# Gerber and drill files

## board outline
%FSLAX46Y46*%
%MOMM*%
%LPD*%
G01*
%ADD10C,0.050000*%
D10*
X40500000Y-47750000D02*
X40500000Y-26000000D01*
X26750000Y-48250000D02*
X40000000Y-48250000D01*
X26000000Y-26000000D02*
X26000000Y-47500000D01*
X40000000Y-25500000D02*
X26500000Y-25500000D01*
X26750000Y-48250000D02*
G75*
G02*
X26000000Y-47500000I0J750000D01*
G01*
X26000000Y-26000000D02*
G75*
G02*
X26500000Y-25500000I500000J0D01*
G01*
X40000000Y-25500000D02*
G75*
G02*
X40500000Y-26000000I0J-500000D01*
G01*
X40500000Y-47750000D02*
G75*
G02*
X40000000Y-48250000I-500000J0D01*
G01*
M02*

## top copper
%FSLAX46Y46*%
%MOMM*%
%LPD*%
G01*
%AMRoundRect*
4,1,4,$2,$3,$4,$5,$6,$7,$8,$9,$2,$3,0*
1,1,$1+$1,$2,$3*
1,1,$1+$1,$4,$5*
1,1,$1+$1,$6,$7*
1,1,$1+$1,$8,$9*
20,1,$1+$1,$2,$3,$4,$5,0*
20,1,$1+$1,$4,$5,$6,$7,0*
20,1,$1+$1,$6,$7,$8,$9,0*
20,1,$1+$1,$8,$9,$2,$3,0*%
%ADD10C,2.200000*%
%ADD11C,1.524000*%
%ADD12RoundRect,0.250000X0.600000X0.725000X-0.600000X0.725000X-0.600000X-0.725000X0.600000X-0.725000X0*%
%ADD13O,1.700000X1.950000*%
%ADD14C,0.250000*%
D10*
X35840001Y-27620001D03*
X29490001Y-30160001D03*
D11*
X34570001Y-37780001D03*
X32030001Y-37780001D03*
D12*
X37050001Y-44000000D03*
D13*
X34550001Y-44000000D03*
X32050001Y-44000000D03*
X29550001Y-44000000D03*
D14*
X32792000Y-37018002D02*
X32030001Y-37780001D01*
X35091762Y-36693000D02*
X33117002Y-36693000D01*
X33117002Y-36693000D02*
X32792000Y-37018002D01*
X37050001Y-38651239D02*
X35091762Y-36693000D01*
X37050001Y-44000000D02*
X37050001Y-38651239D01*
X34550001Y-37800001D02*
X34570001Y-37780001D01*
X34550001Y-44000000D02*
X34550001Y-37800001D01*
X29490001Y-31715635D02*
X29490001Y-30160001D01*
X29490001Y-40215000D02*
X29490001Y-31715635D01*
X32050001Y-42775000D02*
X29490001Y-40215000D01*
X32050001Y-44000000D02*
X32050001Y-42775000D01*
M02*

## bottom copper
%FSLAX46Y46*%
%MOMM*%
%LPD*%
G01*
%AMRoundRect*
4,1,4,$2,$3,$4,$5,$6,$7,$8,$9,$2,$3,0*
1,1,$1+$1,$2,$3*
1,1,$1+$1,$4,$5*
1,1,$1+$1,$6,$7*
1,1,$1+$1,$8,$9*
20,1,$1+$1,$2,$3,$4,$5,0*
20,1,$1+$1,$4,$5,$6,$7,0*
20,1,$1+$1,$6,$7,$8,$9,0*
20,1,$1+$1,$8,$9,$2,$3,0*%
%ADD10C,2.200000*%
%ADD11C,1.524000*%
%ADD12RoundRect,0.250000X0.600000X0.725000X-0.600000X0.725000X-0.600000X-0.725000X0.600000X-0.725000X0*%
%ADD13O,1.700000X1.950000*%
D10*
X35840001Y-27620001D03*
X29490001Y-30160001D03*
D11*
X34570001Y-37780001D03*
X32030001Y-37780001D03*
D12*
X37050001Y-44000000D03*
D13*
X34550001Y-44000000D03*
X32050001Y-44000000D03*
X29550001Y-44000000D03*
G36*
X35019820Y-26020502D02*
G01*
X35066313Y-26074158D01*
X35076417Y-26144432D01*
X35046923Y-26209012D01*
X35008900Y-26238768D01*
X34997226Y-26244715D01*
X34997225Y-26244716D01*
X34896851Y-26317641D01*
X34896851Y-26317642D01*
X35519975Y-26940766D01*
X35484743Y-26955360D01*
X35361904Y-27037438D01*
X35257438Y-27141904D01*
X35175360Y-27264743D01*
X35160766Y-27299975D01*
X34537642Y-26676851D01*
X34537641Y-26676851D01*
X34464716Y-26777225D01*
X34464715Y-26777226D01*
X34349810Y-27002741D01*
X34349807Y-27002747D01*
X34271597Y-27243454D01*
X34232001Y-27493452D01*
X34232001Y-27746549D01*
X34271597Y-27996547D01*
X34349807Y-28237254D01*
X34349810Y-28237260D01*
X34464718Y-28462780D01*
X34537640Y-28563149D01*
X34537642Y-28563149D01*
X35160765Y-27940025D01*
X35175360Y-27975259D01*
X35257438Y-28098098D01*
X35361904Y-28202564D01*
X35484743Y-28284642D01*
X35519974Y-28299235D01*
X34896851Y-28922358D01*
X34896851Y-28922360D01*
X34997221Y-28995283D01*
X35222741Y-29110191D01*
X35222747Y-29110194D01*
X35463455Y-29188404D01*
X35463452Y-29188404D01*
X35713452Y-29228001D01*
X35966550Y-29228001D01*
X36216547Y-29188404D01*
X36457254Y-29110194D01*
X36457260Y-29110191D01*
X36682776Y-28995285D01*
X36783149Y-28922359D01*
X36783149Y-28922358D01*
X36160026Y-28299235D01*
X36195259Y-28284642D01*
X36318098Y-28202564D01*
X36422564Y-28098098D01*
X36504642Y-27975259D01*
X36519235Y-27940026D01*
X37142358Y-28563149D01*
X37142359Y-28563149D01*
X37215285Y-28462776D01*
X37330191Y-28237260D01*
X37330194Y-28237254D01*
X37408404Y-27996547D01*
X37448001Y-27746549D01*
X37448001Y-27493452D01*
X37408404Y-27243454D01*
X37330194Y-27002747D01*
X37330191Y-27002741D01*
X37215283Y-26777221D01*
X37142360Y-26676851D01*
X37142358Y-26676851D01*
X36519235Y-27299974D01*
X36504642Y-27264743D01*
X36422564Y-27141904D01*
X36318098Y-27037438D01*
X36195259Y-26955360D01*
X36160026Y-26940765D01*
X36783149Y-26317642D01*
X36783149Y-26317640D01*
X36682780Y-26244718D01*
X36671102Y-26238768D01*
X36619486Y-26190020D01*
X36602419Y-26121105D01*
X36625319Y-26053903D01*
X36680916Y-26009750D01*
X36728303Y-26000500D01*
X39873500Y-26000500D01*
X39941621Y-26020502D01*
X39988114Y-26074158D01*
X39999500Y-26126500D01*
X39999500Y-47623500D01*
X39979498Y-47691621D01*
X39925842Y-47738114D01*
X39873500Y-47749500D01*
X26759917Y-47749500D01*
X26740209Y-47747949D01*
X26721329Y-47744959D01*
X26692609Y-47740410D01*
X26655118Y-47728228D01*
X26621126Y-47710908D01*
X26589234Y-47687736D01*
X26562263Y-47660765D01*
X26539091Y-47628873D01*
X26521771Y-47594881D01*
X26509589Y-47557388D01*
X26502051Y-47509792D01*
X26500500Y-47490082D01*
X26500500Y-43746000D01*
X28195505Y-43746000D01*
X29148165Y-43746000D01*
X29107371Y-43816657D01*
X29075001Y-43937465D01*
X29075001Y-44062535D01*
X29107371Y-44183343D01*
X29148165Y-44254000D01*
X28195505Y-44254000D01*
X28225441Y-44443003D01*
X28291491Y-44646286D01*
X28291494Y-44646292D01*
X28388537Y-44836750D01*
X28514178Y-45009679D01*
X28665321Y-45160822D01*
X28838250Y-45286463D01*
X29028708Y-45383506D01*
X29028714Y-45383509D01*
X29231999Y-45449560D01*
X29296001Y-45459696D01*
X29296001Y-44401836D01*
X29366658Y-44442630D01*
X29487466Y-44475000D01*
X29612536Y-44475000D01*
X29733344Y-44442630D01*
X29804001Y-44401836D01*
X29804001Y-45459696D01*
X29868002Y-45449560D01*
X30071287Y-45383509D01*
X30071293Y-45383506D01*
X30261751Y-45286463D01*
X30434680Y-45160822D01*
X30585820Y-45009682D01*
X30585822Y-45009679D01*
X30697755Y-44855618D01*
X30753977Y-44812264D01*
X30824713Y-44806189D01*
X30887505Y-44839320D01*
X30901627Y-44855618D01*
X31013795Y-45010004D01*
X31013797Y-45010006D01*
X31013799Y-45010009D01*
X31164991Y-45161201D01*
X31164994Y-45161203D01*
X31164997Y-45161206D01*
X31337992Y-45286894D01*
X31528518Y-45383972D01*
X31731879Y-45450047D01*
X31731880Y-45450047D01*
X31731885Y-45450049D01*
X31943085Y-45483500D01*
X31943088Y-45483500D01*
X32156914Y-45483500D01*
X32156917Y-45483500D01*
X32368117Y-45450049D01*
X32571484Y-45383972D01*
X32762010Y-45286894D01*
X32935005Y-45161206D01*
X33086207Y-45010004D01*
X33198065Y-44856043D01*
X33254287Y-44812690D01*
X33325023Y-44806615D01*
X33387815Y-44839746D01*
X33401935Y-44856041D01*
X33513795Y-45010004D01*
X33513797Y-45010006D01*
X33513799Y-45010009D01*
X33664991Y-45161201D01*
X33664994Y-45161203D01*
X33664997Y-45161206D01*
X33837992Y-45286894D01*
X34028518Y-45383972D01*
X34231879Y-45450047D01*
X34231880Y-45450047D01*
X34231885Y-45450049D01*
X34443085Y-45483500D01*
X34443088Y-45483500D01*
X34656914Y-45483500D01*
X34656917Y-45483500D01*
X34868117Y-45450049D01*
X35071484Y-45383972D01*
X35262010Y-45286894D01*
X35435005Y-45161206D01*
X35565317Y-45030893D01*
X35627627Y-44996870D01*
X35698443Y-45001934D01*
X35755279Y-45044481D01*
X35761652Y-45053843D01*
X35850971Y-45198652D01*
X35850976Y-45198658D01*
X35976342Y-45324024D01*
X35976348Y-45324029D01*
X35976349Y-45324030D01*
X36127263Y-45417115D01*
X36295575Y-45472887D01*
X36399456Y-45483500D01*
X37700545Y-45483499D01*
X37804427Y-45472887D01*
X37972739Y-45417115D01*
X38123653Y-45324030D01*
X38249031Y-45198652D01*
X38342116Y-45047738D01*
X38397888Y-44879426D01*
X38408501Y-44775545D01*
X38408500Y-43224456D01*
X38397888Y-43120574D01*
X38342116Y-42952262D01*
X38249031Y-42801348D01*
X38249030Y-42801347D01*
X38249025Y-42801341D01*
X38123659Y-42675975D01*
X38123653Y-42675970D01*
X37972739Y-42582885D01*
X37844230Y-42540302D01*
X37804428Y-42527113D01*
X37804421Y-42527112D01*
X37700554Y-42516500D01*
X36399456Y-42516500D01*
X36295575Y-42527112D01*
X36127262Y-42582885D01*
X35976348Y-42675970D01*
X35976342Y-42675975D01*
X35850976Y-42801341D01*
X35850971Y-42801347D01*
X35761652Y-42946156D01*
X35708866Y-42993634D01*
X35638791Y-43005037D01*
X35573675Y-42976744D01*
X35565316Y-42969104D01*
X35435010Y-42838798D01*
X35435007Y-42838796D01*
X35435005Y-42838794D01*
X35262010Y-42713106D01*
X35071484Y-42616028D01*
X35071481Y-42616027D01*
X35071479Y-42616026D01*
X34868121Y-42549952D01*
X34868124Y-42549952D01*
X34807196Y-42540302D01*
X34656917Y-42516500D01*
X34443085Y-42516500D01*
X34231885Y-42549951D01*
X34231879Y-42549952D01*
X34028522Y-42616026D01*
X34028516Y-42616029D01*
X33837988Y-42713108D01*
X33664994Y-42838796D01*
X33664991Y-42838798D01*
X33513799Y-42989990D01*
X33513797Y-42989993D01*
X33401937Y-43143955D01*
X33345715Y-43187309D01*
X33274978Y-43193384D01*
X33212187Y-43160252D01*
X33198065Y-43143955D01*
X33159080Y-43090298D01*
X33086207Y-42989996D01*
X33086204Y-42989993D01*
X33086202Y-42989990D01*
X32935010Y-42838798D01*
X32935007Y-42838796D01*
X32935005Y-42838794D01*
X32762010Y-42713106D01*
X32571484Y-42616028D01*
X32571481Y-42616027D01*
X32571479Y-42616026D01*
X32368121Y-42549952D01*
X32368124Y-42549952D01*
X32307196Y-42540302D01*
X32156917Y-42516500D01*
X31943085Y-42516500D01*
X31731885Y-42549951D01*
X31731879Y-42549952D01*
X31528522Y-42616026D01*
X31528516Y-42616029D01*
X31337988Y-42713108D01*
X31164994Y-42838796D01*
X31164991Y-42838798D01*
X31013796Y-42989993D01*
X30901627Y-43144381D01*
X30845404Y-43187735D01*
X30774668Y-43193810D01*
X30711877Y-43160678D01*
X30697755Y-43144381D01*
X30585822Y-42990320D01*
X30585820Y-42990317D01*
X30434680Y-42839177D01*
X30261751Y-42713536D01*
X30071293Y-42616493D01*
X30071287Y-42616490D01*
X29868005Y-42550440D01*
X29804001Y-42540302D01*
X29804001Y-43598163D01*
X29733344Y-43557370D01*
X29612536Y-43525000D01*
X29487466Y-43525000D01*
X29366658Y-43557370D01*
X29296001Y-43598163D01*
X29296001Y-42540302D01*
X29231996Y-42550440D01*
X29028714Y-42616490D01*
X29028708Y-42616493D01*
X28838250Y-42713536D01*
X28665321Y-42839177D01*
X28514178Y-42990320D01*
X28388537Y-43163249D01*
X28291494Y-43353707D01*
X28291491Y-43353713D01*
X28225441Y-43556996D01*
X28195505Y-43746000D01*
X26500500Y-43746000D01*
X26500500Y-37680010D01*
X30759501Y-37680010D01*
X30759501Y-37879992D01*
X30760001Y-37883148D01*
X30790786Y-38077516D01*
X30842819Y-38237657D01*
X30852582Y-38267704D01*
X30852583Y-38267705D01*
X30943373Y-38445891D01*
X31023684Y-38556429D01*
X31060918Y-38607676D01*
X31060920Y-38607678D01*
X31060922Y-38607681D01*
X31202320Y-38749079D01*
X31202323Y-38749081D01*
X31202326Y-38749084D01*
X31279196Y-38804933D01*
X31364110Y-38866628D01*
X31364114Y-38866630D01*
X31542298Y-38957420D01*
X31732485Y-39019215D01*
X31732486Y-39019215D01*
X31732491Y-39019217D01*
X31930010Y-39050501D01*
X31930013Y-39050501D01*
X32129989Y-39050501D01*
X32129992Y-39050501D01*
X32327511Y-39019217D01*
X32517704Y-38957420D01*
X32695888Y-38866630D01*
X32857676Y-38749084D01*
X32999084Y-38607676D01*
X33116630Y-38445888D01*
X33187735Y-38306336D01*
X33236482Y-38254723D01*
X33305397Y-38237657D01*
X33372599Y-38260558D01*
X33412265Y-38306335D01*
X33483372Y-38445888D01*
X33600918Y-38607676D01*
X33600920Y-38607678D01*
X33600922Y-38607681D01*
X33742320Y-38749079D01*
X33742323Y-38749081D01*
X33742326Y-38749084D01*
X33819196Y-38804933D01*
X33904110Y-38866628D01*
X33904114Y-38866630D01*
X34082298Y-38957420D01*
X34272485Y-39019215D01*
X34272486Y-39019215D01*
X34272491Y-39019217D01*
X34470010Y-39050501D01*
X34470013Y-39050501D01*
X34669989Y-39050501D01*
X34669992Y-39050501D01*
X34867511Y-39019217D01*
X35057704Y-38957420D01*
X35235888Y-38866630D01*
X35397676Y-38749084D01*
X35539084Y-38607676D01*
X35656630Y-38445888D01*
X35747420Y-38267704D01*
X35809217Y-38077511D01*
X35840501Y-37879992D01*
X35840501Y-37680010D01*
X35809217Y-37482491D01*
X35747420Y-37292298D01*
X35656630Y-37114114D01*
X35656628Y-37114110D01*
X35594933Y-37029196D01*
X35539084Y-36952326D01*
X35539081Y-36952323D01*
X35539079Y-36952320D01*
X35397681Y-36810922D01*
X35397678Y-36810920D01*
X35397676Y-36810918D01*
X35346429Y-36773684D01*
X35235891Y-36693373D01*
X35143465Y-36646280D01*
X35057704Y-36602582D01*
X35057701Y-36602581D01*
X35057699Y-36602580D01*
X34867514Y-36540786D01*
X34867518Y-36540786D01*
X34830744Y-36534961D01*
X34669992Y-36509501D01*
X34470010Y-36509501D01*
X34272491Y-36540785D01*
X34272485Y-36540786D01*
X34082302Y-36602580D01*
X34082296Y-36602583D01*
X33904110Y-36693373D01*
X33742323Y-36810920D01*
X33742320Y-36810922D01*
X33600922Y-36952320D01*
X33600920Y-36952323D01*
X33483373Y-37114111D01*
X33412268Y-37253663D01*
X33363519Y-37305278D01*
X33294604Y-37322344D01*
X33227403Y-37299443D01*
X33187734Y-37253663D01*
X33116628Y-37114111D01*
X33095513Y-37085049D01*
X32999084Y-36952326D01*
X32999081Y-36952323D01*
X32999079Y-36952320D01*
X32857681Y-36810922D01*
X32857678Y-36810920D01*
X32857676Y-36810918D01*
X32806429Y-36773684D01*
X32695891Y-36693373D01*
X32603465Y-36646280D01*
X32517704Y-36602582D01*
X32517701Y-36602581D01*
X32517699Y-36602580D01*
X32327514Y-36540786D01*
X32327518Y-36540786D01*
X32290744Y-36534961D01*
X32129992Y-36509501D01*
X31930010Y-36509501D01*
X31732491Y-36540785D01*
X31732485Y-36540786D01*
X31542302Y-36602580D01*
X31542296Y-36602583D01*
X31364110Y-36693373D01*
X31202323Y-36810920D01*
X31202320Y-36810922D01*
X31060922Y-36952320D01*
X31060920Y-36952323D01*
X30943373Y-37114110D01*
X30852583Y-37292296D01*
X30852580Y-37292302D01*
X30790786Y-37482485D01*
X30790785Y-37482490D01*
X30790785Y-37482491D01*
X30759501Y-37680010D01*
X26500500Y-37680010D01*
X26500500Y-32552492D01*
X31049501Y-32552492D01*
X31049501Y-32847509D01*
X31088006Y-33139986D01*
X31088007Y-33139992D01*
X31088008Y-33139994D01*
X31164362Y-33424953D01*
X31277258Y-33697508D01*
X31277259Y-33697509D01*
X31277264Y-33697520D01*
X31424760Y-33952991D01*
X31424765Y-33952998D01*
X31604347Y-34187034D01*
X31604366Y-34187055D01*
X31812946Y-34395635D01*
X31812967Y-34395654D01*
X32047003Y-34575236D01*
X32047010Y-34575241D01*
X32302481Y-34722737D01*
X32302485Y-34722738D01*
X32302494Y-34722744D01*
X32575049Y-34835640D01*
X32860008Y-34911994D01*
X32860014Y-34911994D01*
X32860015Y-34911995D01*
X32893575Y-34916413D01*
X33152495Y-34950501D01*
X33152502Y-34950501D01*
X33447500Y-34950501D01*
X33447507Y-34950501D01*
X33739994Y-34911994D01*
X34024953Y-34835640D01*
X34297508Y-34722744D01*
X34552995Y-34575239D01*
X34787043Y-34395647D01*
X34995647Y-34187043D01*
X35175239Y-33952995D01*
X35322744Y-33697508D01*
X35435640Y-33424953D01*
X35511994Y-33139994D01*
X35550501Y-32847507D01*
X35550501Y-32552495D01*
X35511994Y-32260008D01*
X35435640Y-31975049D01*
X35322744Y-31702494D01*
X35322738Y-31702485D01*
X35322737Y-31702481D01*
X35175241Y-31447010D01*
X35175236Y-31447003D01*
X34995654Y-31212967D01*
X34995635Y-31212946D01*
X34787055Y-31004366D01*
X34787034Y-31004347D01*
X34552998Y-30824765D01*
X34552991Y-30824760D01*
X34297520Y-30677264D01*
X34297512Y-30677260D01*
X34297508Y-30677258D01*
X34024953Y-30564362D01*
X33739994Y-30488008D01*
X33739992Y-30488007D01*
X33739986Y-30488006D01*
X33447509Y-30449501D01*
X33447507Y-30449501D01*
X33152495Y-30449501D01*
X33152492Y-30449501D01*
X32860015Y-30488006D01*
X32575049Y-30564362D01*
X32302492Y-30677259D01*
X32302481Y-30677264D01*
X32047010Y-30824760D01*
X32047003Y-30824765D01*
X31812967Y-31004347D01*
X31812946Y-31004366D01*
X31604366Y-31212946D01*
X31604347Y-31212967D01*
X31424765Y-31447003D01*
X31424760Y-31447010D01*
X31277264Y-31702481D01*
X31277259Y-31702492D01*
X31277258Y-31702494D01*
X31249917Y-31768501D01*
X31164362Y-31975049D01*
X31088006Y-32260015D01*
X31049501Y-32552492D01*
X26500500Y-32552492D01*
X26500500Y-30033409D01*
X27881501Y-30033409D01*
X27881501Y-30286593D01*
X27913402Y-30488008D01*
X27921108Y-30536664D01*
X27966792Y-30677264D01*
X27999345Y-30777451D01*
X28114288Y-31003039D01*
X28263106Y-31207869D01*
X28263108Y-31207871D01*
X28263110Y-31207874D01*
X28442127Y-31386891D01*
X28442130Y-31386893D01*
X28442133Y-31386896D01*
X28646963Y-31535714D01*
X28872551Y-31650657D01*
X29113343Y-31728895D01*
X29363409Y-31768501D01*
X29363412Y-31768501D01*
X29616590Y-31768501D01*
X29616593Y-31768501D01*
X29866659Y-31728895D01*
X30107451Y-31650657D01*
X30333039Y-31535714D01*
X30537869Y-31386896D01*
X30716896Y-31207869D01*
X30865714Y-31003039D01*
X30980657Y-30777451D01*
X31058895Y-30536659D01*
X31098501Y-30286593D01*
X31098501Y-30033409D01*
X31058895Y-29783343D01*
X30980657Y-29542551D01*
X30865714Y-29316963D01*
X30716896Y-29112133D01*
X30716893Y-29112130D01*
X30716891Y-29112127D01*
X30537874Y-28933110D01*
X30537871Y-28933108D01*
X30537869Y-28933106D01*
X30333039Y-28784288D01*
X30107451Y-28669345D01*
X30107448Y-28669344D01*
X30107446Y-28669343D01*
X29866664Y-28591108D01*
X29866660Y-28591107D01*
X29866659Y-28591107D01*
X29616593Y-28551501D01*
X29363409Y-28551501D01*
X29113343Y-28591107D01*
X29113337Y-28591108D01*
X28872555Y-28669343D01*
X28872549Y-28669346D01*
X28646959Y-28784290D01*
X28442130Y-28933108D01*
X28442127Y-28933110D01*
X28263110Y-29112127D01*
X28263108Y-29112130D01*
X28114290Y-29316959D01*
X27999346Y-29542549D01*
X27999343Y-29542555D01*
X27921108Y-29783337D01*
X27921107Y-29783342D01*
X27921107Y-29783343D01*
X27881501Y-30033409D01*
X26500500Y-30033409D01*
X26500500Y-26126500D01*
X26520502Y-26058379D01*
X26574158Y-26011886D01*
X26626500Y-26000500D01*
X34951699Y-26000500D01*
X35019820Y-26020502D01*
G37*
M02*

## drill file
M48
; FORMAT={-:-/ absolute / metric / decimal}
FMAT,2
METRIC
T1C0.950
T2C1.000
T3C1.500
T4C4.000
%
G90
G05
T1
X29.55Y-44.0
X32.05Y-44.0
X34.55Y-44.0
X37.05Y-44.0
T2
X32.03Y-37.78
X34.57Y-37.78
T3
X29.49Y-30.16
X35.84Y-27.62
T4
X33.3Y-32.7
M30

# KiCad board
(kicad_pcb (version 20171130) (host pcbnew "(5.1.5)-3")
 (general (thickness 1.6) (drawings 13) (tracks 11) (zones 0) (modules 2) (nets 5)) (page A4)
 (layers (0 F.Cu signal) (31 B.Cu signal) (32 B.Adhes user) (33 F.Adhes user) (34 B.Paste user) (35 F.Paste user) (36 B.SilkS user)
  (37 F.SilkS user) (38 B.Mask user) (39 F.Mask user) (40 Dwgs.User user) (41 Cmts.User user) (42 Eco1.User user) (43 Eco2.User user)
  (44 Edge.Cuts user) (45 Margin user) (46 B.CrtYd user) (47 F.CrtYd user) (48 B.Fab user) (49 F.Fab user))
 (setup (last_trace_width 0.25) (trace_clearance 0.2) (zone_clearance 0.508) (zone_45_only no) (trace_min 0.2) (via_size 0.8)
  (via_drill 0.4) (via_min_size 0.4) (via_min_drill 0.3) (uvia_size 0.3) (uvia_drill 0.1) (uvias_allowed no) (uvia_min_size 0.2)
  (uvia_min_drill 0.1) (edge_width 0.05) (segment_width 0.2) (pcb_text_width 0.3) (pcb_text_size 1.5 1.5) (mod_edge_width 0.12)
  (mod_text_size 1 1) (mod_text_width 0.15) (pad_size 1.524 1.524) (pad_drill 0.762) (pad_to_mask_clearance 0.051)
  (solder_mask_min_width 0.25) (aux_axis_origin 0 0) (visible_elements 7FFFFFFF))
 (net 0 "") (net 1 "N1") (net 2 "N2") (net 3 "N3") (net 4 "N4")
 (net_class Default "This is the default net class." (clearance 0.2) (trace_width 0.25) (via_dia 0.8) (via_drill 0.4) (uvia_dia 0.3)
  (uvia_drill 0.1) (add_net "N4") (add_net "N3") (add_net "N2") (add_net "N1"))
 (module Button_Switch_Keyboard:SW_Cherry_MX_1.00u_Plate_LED (layer F.Cu) (at 35.840001 27.620001)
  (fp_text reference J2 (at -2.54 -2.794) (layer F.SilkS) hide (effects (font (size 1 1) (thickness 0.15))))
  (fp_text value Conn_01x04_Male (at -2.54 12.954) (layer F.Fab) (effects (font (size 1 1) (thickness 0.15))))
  (pad 1 thru_hole circle (at 0 0) (size 2.2 2.2) (drill 1.5) (layers *.Cu *.Mask) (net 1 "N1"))
  (pad 2 thru_hole circle (at -6.35 2.54) (size 2.2 2.2) (drill 1.5) (layers *.Cu *.Mask) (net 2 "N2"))
  (pad "" np_thru_hole circle (at -2.54 5.08) (size 4 4) (drill 4) (layers *.Cu *.Mask))
  (pad 3 thru_hole circle (at -1.27 10.16) (size 1.524 1.524) (drill 1) (layers *.Cu *.Mask) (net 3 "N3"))
  (pad 4 thru_hole circle (at -3.81 10.16) (size 1.524 1.524) (drill 1) (layers *.Cu *.Mask) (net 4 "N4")))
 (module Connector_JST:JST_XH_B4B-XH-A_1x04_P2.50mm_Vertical (layer B.Cu) (at 37.050001 44 180)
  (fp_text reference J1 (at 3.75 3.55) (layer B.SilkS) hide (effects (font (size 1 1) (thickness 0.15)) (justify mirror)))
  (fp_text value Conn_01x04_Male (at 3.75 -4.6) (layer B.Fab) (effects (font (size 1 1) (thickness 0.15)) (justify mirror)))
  (pad 1 thru_hole roundrect (at 0 0 180) (size 1.7 1.95) (drill 0.95) (layers *.Cu *.Mask) (roundrect_rratio 0.147059) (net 4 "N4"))
  (pad 2 thru_hole oval (at 2.5 0 180) (size 1.7 1.95) (drill 0.95) (layers *.Cu *.Mask) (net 3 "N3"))
  (pad 3 thru_hole oval (at 5 0 180) (size 1.7 1.95) (drill 0.95) (layers *.Cu *.Mask) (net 2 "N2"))
  (pad 4 thru_hole oval (at 7.5 0 180) (size 1.7 1.95) (drill 0.95) (layers *.Cu *.Mask) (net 1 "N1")))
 (gr_line (start 40.5 47.75) (end 40.5 26) (layer Edge.Cuts) (width 0.05))
 (gr_line (start 26.75 48.25) (end 40 48.25) (layer Edge.Cuts) (width 0.05))
 (gr_line (start 26 26) (end 26 47.5) (layer Edge.Cuts) (width 0.05))
 (gr_line (start 40 25.5) (end 26.5 25.5) (layer Edge.Cuts) (width 0.05))
 (gr_arc (start 26.75 47.5) (end 26 47.5) (angle -90) (layer Edge.Cuts) (width 0.05))
 (gr_arc (start 26.5 26) (end 26.5 25.5) (angle -90) (layer Edge.Cuts) (width 0.05))
 (gr_arc (start 40 26) (end 40.5 26) (angle -90) (layer Edge.Cuts) (width 0.05))
 (gr_arc (start 40 47.75) (end 40 48.25) (angle -90) (layer Edge.Cuts) (width 0.05))
 (segment (start 32.792 37.018002) (end 32.030001 37.780001) (width 0.25) (layer F.Cu) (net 4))
 (segment (start 35.091762 36.693) (end 33.117002 36.693) (width 0.25) (layer F.Cu) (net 4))
 (segment (start 33.117002 36.693) (end 32.792 37.018002) (width 0.25) (layer F.Cu) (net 4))
 (segment (start 37.050001 38.651239) (end 35.091762 36.693) (width 0.25) (layer F.Cu) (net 4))
 (segment (start 37.050001 44) (end 37.050001 38.651239) (width 0.25) (layer F.Cu) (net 4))
 (segment (start 34.550001 37.800001) (end 34.570001 37.780001) (width 0.25) (layer F.Cu) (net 3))
 (segment (start 34.550001 44) (end 34.550001 37.800001) (width 0.25) (layer F.Cu) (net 3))
 (segment (start 29.490001 31.715635) (end 29.490001 30.160001) (width 0.25) (layer F.Cu) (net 2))
 (segment (start 29.490001 40.215) (end 29.490001 31.715635) (width 0.25) (layer F.Cu) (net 2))
 (segment (start 32.050001 42.775) (end 29.490001 40.215) (width 0.25) (layer F.Cu) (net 2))
 (segment (start 32.050001 44) (end 32.050001 42.775) (width 0.25) (layer F.Cu) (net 2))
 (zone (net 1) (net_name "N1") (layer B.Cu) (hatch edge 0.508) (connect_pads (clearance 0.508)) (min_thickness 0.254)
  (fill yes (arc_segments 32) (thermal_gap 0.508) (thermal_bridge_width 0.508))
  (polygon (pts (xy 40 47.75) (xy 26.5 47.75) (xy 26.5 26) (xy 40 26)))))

